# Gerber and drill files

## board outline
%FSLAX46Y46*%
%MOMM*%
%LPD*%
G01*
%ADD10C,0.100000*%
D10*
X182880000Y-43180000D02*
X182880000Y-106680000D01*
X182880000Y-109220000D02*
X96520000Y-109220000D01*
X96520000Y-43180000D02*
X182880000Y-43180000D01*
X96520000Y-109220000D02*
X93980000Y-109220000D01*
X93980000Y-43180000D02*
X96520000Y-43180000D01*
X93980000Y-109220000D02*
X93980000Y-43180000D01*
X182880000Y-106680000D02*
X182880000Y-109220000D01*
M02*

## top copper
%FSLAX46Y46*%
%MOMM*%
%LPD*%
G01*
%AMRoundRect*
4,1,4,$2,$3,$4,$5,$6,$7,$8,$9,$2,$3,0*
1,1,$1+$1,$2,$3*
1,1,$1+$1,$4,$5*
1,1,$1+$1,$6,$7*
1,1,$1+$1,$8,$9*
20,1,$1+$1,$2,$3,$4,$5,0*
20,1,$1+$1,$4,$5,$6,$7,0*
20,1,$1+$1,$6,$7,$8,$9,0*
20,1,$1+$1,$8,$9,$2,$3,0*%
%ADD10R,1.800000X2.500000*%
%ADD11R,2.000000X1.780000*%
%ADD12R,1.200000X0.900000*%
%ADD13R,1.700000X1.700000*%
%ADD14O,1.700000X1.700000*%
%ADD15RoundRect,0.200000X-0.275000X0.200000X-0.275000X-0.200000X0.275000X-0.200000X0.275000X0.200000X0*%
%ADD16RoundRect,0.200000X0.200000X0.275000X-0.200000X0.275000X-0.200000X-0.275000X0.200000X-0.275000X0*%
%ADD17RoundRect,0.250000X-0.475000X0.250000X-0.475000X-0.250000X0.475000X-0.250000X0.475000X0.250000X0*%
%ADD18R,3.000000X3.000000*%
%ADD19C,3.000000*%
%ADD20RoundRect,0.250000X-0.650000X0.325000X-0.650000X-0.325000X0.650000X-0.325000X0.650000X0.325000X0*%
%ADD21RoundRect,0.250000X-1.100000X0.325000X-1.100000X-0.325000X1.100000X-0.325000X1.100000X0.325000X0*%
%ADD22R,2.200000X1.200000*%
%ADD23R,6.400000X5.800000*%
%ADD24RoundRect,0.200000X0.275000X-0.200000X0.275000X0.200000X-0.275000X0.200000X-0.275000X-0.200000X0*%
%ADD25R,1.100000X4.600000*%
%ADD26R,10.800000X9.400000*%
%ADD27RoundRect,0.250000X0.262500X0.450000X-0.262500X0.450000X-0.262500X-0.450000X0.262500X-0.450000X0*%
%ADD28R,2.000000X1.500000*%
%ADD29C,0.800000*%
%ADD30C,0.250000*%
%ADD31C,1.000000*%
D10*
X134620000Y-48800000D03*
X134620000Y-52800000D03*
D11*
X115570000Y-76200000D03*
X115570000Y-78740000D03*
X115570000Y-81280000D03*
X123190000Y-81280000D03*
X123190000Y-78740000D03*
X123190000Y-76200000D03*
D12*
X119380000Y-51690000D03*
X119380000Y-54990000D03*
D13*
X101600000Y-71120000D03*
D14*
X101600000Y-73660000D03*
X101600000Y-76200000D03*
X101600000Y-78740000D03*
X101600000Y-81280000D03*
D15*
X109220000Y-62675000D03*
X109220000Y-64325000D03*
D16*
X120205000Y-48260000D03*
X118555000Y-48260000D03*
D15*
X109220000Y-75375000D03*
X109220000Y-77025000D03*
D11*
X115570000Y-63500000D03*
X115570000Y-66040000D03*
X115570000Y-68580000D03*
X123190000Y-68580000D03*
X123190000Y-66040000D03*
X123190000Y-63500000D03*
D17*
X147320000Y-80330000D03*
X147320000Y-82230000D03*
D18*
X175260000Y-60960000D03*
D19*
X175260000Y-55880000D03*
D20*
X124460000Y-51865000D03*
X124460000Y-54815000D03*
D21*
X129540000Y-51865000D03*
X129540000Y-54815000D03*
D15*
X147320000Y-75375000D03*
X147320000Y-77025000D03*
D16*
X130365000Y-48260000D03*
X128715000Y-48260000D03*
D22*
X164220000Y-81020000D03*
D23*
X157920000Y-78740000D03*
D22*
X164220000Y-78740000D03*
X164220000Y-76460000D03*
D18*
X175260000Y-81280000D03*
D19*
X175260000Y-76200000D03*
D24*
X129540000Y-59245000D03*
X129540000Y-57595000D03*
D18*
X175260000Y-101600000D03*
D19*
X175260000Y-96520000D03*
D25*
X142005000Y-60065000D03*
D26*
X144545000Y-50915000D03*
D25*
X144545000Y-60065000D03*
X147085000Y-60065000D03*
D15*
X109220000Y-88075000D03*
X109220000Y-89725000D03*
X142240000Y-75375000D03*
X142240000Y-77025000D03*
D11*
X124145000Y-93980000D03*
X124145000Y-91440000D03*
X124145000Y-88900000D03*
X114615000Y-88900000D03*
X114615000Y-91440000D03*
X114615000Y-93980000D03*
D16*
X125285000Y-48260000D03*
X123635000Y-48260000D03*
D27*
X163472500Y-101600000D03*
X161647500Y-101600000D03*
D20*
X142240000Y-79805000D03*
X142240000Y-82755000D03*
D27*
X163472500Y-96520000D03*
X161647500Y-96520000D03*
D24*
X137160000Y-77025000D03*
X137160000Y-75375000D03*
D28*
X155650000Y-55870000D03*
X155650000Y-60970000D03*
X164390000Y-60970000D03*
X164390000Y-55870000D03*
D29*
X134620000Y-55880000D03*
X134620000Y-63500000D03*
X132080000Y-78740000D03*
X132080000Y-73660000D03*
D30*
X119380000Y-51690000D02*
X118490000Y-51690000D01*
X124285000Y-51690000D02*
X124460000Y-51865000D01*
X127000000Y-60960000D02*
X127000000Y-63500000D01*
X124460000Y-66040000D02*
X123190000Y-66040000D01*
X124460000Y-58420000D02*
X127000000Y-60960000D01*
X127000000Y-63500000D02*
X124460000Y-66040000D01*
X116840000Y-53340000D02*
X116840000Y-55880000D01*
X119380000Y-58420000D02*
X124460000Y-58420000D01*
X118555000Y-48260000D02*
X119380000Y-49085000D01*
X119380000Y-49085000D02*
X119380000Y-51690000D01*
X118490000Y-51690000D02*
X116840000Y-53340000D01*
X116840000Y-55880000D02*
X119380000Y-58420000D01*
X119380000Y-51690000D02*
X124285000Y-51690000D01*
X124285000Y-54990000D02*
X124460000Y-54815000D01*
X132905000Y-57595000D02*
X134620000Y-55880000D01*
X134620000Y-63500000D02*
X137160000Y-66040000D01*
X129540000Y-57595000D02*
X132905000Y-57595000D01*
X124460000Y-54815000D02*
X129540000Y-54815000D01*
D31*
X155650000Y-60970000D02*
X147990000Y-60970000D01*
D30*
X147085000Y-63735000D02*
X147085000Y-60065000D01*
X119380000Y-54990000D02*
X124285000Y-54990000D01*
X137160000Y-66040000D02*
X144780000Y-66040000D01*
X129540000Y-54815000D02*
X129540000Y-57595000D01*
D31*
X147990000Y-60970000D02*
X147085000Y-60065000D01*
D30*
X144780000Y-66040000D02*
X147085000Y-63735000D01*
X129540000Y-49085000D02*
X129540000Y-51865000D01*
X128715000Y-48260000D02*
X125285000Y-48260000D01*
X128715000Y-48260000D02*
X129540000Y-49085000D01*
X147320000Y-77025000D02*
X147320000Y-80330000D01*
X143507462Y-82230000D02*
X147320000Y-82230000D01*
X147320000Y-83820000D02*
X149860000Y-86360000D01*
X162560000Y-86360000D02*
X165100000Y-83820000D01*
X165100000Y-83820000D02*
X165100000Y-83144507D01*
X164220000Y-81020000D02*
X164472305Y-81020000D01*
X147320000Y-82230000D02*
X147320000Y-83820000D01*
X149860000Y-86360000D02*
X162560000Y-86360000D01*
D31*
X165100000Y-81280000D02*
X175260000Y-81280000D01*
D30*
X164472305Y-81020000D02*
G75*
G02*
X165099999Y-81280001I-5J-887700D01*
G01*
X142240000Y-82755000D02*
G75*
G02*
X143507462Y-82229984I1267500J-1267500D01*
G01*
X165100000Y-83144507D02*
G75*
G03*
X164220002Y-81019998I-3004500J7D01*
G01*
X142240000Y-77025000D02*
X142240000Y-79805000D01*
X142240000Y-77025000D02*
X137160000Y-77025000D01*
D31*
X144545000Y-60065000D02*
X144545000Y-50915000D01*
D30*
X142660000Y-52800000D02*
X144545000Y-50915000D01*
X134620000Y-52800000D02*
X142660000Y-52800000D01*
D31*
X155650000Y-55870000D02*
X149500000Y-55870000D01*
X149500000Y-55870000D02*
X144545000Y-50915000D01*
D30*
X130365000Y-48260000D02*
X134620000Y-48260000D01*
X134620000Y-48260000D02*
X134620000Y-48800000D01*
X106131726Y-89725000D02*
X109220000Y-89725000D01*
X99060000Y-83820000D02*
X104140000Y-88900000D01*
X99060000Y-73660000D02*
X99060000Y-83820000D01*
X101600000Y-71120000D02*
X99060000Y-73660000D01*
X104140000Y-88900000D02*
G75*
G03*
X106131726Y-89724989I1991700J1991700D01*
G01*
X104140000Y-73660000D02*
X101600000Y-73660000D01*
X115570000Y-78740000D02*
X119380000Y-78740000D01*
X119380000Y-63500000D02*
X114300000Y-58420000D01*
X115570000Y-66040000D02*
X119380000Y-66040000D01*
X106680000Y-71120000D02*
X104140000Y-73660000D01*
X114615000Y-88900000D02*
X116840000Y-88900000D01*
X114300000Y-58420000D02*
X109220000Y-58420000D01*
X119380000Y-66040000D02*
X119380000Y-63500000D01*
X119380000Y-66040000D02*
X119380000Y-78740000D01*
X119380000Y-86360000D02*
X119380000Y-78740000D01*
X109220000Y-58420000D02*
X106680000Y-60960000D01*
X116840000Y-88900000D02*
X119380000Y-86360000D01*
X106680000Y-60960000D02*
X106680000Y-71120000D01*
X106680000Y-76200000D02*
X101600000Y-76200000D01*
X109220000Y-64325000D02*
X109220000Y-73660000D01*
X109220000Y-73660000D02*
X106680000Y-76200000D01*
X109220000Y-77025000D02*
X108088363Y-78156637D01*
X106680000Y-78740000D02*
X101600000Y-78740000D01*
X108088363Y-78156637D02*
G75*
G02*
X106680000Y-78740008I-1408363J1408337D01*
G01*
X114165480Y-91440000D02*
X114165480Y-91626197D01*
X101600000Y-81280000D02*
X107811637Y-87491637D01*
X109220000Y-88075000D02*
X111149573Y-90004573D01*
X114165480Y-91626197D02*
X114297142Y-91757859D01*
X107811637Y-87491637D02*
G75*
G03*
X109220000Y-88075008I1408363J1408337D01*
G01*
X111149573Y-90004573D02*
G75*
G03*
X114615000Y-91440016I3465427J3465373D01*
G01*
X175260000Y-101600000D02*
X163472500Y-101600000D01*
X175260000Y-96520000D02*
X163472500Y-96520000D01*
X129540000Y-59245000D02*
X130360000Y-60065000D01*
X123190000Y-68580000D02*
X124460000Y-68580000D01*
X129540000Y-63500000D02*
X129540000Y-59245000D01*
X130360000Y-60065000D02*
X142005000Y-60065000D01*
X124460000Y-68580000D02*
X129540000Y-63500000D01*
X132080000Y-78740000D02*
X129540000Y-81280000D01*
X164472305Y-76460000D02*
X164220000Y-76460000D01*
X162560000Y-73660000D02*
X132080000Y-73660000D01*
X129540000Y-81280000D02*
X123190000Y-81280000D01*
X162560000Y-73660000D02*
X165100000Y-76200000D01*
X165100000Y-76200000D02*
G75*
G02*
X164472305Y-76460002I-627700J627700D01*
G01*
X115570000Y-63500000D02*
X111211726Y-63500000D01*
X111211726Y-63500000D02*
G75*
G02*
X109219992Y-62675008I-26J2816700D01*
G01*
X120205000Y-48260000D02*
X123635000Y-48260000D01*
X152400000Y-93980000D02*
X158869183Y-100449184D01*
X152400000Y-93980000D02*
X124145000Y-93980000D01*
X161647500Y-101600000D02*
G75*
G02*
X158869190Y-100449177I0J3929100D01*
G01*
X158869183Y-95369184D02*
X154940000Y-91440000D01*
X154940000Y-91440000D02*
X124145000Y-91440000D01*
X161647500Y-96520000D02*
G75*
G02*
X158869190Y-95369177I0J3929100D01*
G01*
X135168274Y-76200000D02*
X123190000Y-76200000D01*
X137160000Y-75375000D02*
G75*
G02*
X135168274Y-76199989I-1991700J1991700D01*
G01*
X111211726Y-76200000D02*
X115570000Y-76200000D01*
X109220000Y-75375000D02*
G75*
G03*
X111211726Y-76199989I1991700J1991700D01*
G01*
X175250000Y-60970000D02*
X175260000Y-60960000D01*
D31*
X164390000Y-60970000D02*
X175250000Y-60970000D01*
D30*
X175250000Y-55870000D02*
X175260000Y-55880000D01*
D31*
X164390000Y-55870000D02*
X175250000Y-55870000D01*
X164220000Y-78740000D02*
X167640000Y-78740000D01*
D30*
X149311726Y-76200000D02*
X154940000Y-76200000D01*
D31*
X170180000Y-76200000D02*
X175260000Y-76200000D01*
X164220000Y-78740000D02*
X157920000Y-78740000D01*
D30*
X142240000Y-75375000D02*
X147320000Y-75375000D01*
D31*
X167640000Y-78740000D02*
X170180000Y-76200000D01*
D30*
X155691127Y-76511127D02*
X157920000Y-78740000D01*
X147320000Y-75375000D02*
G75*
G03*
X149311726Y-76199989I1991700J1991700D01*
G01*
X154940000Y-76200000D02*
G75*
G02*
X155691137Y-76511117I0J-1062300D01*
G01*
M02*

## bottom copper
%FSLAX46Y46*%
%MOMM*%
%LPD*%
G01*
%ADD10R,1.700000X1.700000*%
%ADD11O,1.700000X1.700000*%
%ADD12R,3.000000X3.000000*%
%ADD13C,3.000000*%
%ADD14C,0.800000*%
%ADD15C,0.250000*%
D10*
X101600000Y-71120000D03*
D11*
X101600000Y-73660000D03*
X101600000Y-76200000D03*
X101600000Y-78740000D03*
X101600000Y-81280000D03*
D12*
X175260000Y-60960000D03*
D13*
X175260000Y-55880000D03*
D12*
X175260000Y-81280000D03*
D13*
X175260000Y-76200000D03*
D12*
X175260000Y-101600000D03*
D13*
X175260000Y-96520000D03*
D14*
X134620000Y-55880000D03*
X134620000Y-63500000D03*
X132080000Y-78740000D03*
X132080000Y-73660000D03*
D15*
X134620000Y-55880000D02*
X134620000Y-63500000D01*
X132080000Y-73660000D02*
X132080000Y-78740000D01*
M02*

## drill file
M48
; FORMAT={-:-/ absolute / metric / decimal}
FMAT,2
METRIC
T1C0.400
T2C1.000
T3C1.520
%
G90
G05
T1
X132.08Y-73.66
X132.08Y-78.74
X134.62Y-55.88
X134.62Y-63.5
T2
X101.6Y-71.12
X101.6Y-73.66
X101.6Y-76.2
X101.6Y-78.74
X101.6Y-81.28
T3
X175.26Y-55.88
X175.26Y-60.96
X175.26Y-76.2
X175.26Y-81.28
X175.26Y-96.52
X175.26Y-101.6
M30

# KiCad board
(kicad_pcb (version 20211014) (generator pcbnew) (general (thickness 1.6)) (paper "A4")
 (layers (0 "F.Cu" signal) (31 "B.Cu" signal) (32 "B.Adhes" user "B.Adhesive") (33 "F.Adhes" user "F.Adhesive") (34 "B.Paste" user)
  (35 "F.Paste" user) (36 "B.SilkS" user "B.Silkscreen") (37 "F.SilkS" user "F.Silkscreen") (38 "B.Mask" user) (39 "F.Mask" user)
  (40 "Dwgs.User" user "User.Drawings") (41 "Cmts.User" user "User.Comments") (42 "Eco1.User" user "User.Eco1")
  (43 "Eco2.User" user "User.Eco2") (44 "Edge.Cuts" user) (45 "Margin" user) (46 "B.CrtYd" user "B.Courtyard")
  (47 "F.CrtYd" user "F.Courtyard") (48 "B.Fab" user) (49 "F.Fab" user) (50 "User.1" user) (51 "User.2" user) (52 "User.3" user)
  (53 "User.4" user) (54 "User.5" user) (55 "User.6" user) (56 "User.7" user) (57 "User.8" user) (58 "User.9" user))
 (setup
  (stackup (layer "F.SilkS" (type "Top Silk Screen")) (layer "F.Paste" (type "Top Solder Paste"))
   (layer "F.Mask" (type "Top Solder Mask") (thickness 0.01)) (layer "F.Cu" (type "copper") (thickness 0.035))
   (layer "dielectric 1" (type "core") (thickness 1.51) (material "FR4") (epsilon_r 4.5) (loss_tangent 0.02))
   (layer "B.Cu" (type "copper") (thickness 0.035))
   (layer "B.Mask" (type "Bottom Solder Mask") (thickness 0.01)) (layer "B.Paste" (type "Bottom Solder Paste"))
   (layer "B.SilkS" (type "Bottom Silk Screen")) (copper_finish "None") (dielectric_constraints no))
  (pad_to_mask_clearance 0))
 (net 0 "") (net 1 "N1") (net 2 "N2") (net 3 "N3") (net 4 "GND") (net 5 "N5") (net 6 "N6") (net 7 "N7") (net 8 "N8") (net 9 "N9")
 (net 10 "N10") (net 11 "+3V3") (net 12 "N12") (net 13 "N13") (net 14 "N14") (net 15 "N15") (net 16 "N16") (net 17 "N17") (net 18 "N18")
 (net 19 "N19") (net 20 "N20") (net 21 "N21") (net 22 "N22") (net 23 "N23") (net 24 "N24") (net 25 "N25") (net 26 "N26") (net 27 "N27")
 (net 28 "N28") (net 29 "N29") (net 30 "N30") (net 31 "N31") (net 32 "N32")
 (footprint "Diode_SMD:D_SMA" (layer "F.Cu") (at 134.62 50.8 -90)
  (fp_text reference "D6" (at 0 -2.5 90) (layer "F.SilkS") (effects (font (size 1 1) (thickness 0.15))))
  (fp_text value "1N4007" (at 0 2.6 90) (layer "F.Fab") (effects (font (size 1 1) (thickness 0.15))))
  (pad "1" smd rect locked (at -2 0 270) (size 2.5 1.8) (layers "F.Cu" "F.Paste" "F.Mask") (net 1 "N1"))
  (pad "2" smd rect locked (at 2 0 270) (size 2.5 1.8) (layers "F.Cu" "F.Paste" "F.Mask") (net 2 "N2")))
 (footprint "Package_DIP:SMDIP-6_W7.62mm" (layer "F.Cu") (at 119.38 78.74)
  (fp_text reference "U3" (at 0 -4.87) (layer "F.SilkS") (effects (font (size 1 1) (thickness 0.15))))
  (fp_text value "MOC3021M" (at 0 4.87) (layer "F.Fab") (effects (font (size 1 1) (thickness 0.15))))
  (pad "1" smd rect locked (at -3.81 -2.54) (size 2 1.78) (layers "F.Cu" "F.Paste" "F.Mask") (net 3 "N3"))
  (pad "2" smd rect locked (at -3.81 0) (size 2 1.78) (layers "F.Cu" "F.Paste" "F.Mask") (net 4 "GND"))
  (pad "3" smd rect locked (at -3.81 2.54) (size 2 1.78) (layers "F.Cu" "F.Paste" "F.Mask") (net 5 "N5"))
  (pad "4" smd rect locked (at 3.81 2.54) (size 2 1.78) (layers "F.Cu" "F.Paste" "F.Mask") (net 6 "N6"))
  (pad "5" smd rect locked (at 3.81 0) (size 2 1.78) (layers "F.Cu" "F.Paste" "F.Mask") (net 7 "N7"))
  (pad "6" smd rect locked (at 3.81 -2.54) (size 2 1.78) (layers "F.Cu" "F.Paste" "F.Mask") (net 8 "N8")))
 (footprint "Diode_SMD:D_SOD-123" (layer "F.Cu") (at 119.38 53.34 -90)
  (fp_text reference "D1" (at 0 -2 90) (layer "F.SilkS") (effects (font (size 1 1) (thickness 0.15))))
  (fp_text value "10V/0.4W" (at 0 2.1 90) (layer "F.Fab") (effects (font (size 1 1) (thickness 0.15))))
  (pad "1" smd rect locked (at -1.65 0 270) (size 0.9 1.2) (layers "F.Cu" "F.Paste" "F.Mask") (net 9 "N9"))
  (pad "2" smd rect locked (at 1.65 0 270) (size 0.9 1.2) (layers "F.Cu" "F.Paste" "F.Mask") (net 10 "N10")))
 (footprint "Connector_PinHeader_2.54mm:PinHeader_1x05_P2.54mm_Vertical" (layer "F.Cu") (at 101.6 71.12)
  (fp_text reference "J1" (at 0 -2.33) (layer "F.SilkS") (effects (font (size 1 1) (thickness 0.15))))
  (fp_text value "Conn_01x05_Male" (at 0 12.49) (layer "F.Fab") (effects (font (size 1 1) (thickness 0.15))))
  (pad "1" thru_hole rect locked (at 0 0) (size 1.7 1.7) (drill 1) (layers *.Cu *.Mask) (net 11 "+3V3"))
  (pad "2" thru_hole oval locked (at 0 2.54) (size 1.7 1.7) (drill 1) (layers *.Cu *.Mask) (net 4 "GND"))
  (pad "3" thru_hole oval locked (at 0 5.08) (size 1.7 1.7) (drill 1) (layers *.Cu *.Mask) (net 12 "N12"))
  (pad "4" thru_hole oval locked (at 0 7.62) (size 1.7 1.7) (drill 1) (layers *.Cu *.Mask) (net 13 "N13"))
  (pad "5" thru_hole oval locked (at 0 10.16) (size 1.7 1.7) (drill 1) (layers *.Cu *.Mask) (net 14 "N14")))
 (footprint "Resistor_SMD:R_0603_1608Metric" (layer "F.Cu") (at 109.22 63.5 -90)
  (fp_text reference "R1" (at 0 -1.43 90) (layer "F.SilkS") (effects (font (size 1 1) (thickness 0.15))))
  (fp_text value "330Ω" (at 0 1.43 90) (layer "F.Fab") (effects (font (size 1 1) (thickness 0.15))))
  (pad "1" smd roundrect locked (at -0.825 0 270) (size 0.8 0.95) (layers "F.Cu" "F.Paste" "F.Mask") (roundrect_rratio 0.25) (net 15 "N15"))
  (pad "2" smd roundrect locked (at 0.825 0 270) (size 0.8 0.95) (layers "F.Cu" "F.Paste" "F.Mask") (roundrect_rratio 0.25) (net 12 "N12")))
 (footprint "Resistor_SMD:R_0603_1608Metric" (layer "F.Cu") (at 119.38 48.26 180)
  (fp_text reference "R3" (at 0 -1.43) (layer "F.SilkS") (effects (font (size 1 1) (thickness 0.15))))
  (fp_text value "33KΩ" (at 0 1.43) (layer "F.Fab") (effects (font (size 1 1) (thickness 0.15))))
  (pad "1" smd roundrect locked (at -0.825 0 180) (size 0.8 0.95) (layers "F.Cu" "F.Paste" "F.Mask") (roundrect_rratio 0.25) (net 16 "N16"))
  (pad "2" smd roundrect locked (at 0.825 0 180) (size 0.8 0.95) (layers "F.Cu" "F.Paste" "F.Mask") (roundrect_rratio 0.25) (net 9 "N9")))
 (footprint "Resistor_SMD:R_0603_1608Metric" (layer "F.Cu") (at 109.22 76.2 -90)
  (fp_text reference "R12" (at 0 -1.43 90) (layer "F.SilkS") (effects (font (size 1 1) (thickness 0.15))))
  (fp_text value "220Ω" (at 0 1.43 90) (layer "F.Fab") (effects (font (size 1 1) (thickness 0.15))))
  (pad "1" smd roundrect locked (at -0.825 0 270) (size 0.8 0.95) (layers "F.Cu" "F.Paste" "F.Mask") (roundrect_rratio 0.25) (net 3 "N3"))
  (pad "2" smd roundrect locked (at 0.825 0 270) (size 0.8 0.95) (layers "F.Cu" "F.Paste" "F.Mask") (roundrect_rratio 0.25) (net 13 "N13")))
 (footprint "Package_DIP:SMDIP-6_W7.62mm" (layer "F.Cu") (at 119.38 66.04)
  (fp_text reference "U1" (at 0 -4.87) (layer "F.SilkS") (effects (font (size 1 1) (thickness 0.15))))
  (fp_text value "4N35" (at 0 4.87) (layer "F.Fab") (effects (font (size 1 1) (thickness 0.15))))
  (pad "1" smd rect locked (at -3.81 -2.54) (size 2 1.78) (layers "F.Cu" "F.Paste" "F.Mask") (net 15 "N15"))
  (pad "2" smd rect locked (at -3.81 0) (size 2 1.78) (layers "F.Cu" "F.Paste" "F.Mask") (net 4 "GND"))
  (pad "3" smd rect locked (at -3.81 2.54) (size 2 1.78) (layers "F.Cu" "F.Paste" "F.Mask") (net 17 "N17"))
  (pad "4" smd rect locked (at 3.81 2.54) (size 2 1.78) (layers "F.Cu" "F.Paste" "F.Mask") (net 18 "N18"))
  (pad "5" smd rect locked (at 3.81 0) (size 2 1.78) (layers "F.Cu" "F.Paste" "F.Mask") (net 9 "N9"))
  (pad "6" smd rect locked (at 3.81 -2.54) (size 2 1.78) (layers "F.Cu" "F.Paste" "F.Mask") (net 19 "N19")))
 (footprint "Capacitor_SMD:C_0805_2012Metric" (layer "F.Cu") (at 147.32 81.28 -90)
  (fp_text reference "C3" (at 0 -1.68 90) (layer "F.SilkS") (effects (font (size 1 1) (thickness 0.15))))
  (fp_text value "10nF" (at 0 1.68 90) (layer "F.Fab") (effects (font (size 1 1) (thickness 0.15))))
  (pad "1" smd roundrect locked (at -0.95 0 270) (size 1 1.45) (layers "F.Cu" "F.Paste" "F.Mask") (roundrect_rratio 0.25) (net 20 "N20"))
  (pad "2" smd roundrect locked (at 0.95 0 270) (size 1 1.45) (layers "F.Cu" "F.Paste" "F.Mask") (roundrect_rratio 0.25) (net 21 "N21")))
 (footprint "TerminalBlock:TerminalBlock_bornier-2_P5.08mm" (layer "F.Cu") (at 175.26 60.96 90)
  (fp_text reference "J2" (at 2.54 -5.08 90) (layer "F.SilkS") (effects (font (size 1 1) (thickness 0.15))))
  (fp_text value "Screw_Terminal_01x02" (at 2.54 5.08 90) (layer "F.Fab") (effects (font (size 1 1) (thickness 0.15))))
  (pad "1" thru_hole rect locked (at 0 0 90) (size 3 3) (drill 1.52) (layers *.Cu *.Mask) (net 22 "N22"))
  (pad "2" thru_hole circle locked (at 5.08 0 90) (size 3 3) (drill 1.52) (layers *.Cu *.Mask) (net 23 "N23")))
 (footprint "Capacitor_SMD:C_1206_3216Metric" (layer "F.Cu") (at 124.46 53.34 -90)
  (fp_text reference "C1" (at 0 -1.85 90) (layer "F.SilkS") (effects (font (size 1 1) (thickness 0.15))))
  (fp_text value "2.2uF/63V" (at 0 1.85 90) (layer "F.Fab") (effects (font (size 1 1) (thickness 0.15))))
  (pad "1" smd roundrect locked (at -1.475 0 270) (size 1.15 1.8) (layers "F.Cu" "F.Paste" "F.Mask") (roundrect_rratio 0.2173913043)
   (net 9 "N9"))
  (pad "2" smd roundrect locked (at 1.475 0 270) (size 1.15 1.8) (layers "F.Cu" "F.Paste" "F.Mask") (roundrect_rratio 0.2173913043)
   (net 10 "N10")))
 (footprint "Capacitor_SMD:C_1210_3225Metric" (layer "F.Cu") (at 129.54 53.34 -90)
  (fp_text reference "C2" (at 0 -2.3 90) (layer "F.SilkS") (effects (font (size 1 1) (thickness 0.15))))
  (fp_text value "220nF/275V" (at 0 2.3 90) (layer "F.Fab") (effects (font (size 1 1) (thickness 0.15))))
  (pad "1" smd roundrect locked (at -1.475 0 270) (size 1.15 2.7) (layers "F.Cu" "F.Paste" "F.Mask") (roundrect_rratio 0.2173913043)
   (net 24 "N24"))
  (pad "2" smd roundrect locked (at 1.475 0 270) (size 1.15 2.7) (layers "F.Cu" "F.Paste" "F.Mask") (roundrect_rratio 0.2173913043)
   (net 10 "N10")))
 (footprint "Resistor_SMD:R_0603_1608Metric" (layer "F.Cu") (at 147.32 76.2 -90)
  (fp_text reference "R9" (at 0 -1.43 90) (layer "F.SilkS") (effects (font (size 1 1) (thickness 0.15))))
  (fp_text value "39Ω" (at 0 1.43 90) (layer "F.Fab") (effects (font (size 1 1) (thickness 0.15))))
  (pad "1" smd roundrect locked (at -0.825 0 270) (size 0.8 0.95) (layers "F.Cu" "F.Paste" "F.Mask") (roundrect_rratio 0.25) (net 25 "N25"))
  (pad "2" smd roundrect locked (at 0.825 0 270) (size 0.8 0.95) (layers "F.Cu" "F.Paste" "F.Mask") (roundrect_rratio 0.25) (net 20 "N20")))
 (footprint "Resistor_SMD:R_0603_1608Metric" (layer "F.Cu") (at 129.54 48.26 180)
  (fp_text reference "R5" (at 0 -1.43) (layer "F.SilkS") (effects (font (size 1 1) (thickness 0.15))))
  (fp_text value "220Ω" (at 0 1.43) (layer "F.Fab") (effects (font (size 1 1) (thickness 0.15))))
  (pad "1" smd roundrect locked (at -0.825 0 180) (size 0.8 0.95) (layers "F.Cu" "F.Paste" "F.Mask") (roundrect_rratio 0.25) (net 1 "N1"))
  (pad "2" smd roundrect locked (at 0.825 0 180) (size 0.8 0.95) (layers "F.Cu" "F.Paste" "F.Mask") (roundrect_rratio 0.25) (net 24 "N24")))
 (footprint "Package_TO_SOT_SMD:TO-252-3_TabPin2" (layer "F.Cu") (at 160.02 78.74 180)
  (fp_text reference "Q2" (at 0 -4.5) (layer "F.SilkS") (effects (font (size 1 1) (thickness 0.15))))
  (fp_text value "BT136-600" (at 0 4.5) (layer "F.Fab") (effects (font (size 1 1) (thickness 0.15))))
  (pad "" smd rect locked (at 0.425 1.525 180) (size 3.05 2.75) (layers "F.Paste"))
  (pad "" smd rect locked (at 3.775 -1.525 180) (size 3.05 2.75) (layers "F.Paste"))
  (pad "" smd rect locked (at 0.425 -1.525 180) (size 3.05 2.75) (layers "F.Paste"))
  (pad "" smd rect locked (at 3.775 1.525 180) (size 3.05 2.75) (layers "F.Paste"))
  (pad "1" smd rect locked (at -4.2 -2.28 180) (size 2.2 1.2) (layers "F.Cu" "F.Paste" "F.Mask") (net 21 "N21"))
  (pad "2" smd rect locked (at 2.1 0 180) (size 6.4 5.8) (layers "F.Cu" "F.Mask") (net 25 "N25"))
  (pad "2" smd rect locked (at -4.2 0 180) (size 2.2 1.2) (layers "F.Cu" "F.Paste" "F.Mask") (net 25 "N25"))
  (pad "3" smd rect locked (at -4.2 2.28 180) (size 2.2 1.2) (layers "F.Cu" "F.Paste" "F.Mask") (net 6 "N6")))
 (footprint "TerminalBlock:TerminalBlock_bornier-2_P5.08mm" (layer "F.Cu") (at 175.26 81.28 90)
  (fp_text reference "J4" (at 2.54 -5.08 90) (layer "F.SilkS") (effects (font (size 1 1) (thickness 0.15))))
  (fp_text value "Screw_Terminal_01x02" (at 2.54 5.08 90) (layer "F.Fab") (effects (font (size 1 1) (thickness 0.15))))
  (pad "1" thru_hole rect locked (at 0 0 90) (size 3 3) (drill 1.52) (layers *.Cu *.Mask) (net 21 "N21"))
  (pad "2" thru_hole circle locked (at 5.08 0 90) (size 3 3) (drill 1.52) (layers *.Cu *.Mask) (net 25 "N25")))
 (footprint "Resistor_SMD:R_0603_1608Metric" (layer "F.Cu") (at 129.54 58.42 90)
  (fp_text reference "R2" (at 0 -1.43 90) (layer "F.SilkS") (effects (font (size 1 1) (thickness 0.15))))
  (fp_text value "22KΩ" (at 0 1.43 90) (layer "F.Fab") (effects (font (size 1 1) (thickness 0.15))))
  (pad "1" smd roundrect locked (at -0.825 0 90) (size 0.8 0.95) (layers "F.Cu" "F.Paste" "F.Mask") (roundrect_rratio 0.25) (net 18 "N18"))
  (pad "2" smd roundrect locked (at 0.825 0 90) (size 0.8 0.95) (layers "F.Cu" "F.Paste" "F.Mask") (roundrect_rratio 0.25) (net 10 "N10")))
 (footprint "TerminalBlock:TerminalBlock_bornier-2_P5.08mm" (layer "F.Cu") (at 175.26 101.6 90)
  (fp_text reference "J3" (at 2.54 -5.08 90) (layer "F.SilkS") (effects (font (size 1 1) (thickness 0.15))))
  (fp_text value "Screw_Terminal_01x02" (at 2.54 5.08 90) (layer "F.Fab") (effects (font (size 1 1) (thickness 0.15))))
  (pad "1" thru_hole rect locked (at 0 0 90) (size 3 3) (drill 1.52) (layers *.Cu *.Mask) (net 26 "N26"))
  (pad "2" thru_hole circle locked (at 5.08 0 90) (size 3 3) (drill 1.52) (layers *.Cu *.Mask) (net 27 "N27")))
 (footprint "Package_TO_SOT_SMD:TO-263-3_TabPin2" (layer "F.Cu") (at 144.545 54.29 90)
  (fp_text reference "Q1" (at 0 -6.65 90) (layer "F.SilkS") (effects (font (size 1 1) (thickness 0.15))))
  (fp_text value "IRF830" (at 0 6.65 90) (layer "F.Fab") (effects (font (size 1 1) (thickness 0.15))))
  (pad "" smd rect locked (at 5.8 2.775 90) (size 4.55 5.25) (layers "F.Paste"))
  (pad "" smd rect locked (at 0.95 -2.775 90) (size 4.55 5.25) (layers "F.Paste"))
  (pad "" smd rect locked (at 0.95 2.775 90) (size 4.55 5.25) (layers "F.Paste"))
  (pad "" smd rect locked (at 5.8 -2.775 90) (size 4.55 5.25) (layers "F.Paste"))
  (pad "1" smd rect locked (at -5.775 -2.54 90) (size 4.6 1.1) (layers "F.Cu" "F.Paste" "F.Mask") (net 18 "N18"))
  (pad "2" smd rect locked (at 3.375 0 90) (size 9.4 10.8) (layers "F.Cu" "F.Mask") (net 2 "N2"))
  (pad "2" smd rect locked (at -5.775 0 90) (size 4.6 1.1) (layers "F.Cu" "F.Paste" "F.Mask") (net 2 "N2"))
  (pad "3" smd rect locked (at -5.775 2.54 90) (size 4.6 1.1) (layers "F.Cu" "F.Paste" "F.Mask") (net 10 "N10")))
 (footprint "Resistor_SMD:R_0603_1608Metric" (layer "F.Cu") (at 109.22 88.9 -90)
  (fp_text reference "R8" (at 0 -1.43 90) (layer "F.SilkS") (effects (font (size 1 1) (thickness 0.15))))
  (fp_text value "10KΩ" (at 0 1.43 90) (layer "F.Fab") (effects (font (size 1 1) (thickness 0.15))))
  (pad "1" smd roundrect locked (at -0.825 0 270) (size 0.8 0.95) (layers "F.Cu" "F.Paste" "F.Mask") (roundrect_rratio 0.25) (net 14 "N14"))
  (pad "2" smd roundrect locked (at 0.825 0 270) (size 0.8 0.95) (layers "F.Cu" "F.Paste" "F.Mask") (roundrect_rratio 0.25) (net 11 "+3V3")))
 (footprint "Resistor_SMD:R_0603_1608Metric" (layer "F.Cu") (at 142.24 76.2 -90)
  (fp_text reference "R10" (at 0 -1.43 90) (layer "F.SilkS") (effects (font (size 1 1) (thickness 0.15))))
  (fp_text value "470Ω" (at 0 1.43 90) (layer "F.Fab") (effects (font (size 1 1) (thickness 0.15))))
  (pad "1" smd roundrect locked (at -0.825 0 270) (size 0.8 0.95) (layers "F.Cu" "F.Paste" "F.Mask") (roundrect_rratio 0.25) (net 25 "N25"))
  (pad "2" smd roundrect locked (at 0.825 0 270) (size 0.8 0.95) (layers "F.Cu" "F.Paste" "F.Mask") (roundrect_rratio 0.25) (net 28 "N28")))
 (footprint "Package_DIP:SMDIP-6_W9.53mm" (layer "F.Cu") (at 119.38 91.44 180)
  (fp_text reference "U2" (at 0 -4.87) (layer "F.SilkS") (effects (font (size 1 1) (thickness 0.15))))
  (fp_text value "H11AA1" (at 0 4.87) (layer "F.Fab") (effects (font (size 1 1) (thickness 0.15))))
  (pad "1" smd rect locked (at -4.765 -2.54 180) (size 2 1.78) (layers "F.Cu" "F.Paste" "F.Mask") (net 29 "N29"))
  (pad "2" smd rect locked (at -4.765 0 180) (size 2 1.78) (layers "F.Cu" "F.Paste" "F.Mask") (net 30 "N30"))
  (pad "3" smd rect locked (at -4.765 2.54 180) (size 2 1.78) (layers "F.Cu" "F.Paste" "F.Mask") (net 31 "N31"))
  (pad "4" smd rect locked (at 4.765 2.54 180) (size 2 1.78) (layers "F.Cu" "F.Paste" "F.Mask") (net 4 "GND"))
  (pad "5" smd rect locked (at 4.765 0 180) (size 2 1.78) (layers "F.Cu" "F.Paste" "F.Mask") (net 14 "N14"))
  (pad "6" smd rect locked (at 4.765 -2.54 180) (size 2 1.78) (layers "F.Cu" "F.Paste" "F.Mask") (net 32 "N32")))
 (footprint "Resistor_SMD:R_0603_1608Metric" (layer "F.Cu") (at 124.46 48.26 180)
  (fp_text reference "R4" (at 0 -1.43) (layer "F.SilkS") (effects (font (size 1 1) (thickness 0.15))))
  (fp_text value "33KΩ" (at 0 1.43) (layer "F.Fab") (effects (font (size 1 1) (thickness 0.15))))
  (pad "1" smd roundrect locked (at -0.825 0 180) (size 0.8 0.95) (layers "F.Cu" "F.Paste" "F.Mask") (roundrect_rratio 0.25) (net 24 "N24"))
  (pad "2" smd roundrect locked (at 0.825 0 180) (size 0.8 0.95) (layers "F.Cu" "F.Paste" "F.Mask") (roundrect_rratio 0.25) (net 16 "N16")))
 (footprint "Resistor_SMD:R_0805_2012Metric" (layer "F.Cu") (at 162.56 101.6 180)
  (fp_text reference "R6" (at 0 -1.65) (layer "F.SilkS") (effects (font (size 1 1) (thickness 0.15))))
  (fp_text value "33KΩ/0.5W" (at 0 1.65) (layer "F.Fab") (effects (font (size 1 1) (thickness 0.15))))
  (pad "1" smd roundrect locked (at -0.9125 0 180) (size 1.025 1.4) (layers "F.Cu" "F.Paste" "F.Mask") (roundrect_rratio 0.243902439)
   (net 26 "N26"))
  (pad "2" smd roundrect locked (at 0.9125 0 180) (size 1.025 1.4) (layers "F.Cu" "F.Paste" "F.Mask") (roundrect_rratio 0.243902439)
   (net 29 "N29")))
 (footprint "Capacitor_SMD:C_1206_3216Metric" (layer "F.Cu") (at 142.24 81.28 -90)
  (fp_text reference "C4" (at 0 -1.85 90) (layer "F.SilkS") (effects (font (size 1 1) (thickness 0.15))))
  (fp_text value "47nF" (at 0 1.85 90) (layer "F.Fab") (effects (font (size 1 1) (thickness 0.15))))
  (pad "1" smd roundrect locked (at -1.475 0 270) (size 1.15 1.8) (layers "F.Cu" "F.Paste" "F.Mask") (roundrect_rratio 0.2173913043)
   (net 28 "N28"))
  (pad "2" smd roundrect locked (at 1.475 0 270) (size 1.15 1.8) (layers "F.Cu" "F.Paste" "F.Mask") (roundrect_rratio 0.2173913043)
   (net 21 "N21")))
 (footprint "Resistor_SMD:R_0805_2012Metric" (layer "F.Cu") (at 162.56 96.52 180)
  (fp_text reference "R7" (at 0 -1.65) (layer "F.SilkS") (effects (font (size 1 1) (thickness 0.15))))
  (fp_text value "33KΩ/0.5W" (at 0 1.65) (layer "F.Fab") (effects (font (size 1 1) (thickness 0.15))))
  (pad "1" smd roundrect locked (at -0.9125 0 180) (size 1.025 1.4) (layers "F.Cu" "F.Paste" "F.Mask") (roundrect_rratio 0.243902439)
   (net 27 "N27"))
  (pad "2" smd roundrect locked (at 0.9125 0 180) (size 1.025 1.4) (layers "F.Cu" "F.Paste" "F.Mask") (roundrect_rratio 0.243902439)
   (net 30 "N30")))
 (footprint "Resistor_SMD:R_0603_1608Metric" (layer "F.Cu") (at 137.16 76.2 90)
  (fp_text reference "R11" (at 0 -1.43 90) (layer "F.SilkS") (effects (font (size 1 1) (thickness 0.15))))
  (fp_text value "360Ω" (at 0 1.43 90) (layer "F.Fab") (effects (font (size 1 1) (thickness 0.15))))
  (pad "1" smd roundrect locked (at -0.825 0 90) (size 0.8 0.95) (layers "F.Cu" "F.Paste" "F.Mask") (roundrect_rratio 0.25) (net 28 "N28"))
  (pad "2" smd roundrect locked (at 0.825 0 90) (size 0.8 0.95) (layers "F.Cu" "F.Paste" "F.Mask") (roundrect_rratio 0.25) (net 8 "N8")))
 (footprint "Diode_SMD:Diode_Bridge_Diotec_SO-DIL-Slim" (layer "F.Cu") (at 160.02 58.42)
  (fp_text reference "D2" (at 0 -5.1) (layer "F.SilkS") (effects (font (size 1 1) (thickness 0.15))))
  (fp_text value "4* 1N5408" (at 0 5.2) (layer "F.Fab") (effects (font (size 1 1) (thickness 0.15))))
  (pad "1" smd rect locked (at -4.37 -2.55) (size 2 1.5) (layers "F.Cu" "F.Paste" "F.Mask") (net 2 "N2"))
  (pad "2" smd rect locked (at -4.37 2.55) (size 2 1.5) (layers "F.Cu" "F.Paste" "F.Mask") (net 10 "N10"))
  (pad "3" smd rect locked (at 4.37 2.55) (size 2 1.5) (layers "F.Cu" "F.Paste" "F.Mask") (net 22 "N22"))
  (pad "4" smd rect locked (at 4.37 -2.55) (size 2 1.5) (layers "F.Cu" "F.Paste" "F.Mask") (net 23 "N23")))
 (gr_line (start 182.88 43.18) (end 182.88 106.68) (layer "Edge.Cuts") (width 0.1))
 (gr_line (start 182.88 109.22) (end 96.52 109.22) (layer "Edge.Cuts") (width 0.1))
 (gr_line (start 96.52 43.18) (end 182.88 43.18) (layer "Edge.Cuts") (width 0.1))
 (gr_line (start 96.52 109.22) (end 93.98 109.22) (layer "Edge.Cuts") (width 0.1))
 (gr_line (start 93.98 43.18) (end 96.52 43.18) (layer "Edge.Cuts") (width 0.1))
 (gr_line (start 93.98 109.22) (end 93.98 43.18) (layer "Edge.Cuts") (width 0.1))
 (gr_line (start 182.88 106.68) (end 182.88 109.22) (layer "Edge.Cuts") (width 0.1))
 (segment (start 119.38 51.69) (end 118.49 51.69) (width 0.25) (layer "F.Cu") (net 9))
 (segment (start 124.285 51.69) (end 124.46 51.865) (width 0.25) (layer "F.Cu") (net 9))
 (segment (start 127 60.96) (end 127 63.5) (width 0.25) (layer "F.Cu") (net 9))
 (segment (start 124.46 66.04) (end 123.19 66.04) (width 0.25) (layer "F.Cu") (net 9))
 (segment (start 124.46 58.42) (end 127 60.96) (width 0.25) (layer "F.Cu") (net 9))
 (segment (start 127 63.5) (end 124.46 66.04) (width 0.25) (layer "F.Cu") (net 9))
 (segment (start 116.84 53.34) (end 116.84 55.88) (width 0.25) (layer "F.Cu") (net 9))
 (segment (start 119.38 58.42) (end 124.46 58.42) (width 0.25) (layer "F.Cu") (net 9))
 (segment (start 118.555 48.26) (end 119.38 49.085) (width 0.25) (layer "F.Cu") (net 9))
 (segment (start 119.38 49.085) (end 119.38 51.69) (width 0.25) (layer "F.Cu") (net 9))
 (segment (start 118.49 51.69) (end 116.84 53.34) (width 0.25) (layer "F.Cu") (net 9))
 (segment (start 116.84 55.88) (end 119.38 58.42) (width 0.25) (layer "F.Cu") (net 9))
 (segment (start 119.38 51.69) (end 124.285 51.69) (width 0.25) (layer "F.Cu") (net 9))
 (segment (start 124.285 54.99) (end 124.46 54.815) (width 0.25) (layer "F.Cu") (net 10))
 (segment (start 132.905 57.595) (end 134.62 55.88) (width 0.25) (layer "F.Cu") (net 10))
 (segment (start 134.62 63.5) (end 137.16 66.04) (width 0.25) (layer "F.Cu") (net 10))
 (segment (start 129.54 57.595) (end 132.905 57.595) (width 0.25) (layer "F.Cu") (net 10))
 (segment (start 124.46 54.815) (end 129.54 54.815) (width 0.25) (layer "F.Cu") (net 10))
 (segment (start 155.65 60.97) (end 147.99 60.97) (width 1) (layer "F.Cu") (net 10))
 (segment (start 147.085 63.735) (end 147.085 60.065) (width 0.25) (layer "F.Cu") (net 10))
 (segment (start 119.38 54.99) (end 124.285 54.99) (width 0.25) (layer "F.Cu") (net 10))
 (segment (start 137.16 66.04) (end 144.78 66.04) (width 0.25) (layer "F.Cu") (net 10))
 (segment (start 129.54 54.815) (end 129.54 57.595) (width 0.25) (layer "F.Cu") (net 10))
 (segment (start 147.99 60.97) (end 147.085 60.065) (width 1) (layer "F.Cu") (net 10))
 (segment (start 144.78 66.04) (end 147.085 63.735) (width 0.25) (layer "F.Cu") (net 10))
 (via (at 134.62 55.88) (size 0.8) (drill 0.4) (layers "F.Cu" "B.Cu") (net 10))
 (via (at 134.62 63.5) (size 0.8) (drill 0.4) (layers "F.Cu" "B.Cu") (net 10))
 (segment (start 134.62 55.88) (end 134.62 63.5) (width 0.25) (layer "B.Cu") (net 10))
 (segment (start 129.54 49.085) (end 129.54 51.865) (width 0.25) (layer "F.Cu") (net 24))
 (segment (start 128.715 48.26) (end 125.285 48.26) (width 0.25) (layer "F.Cu") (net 24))
 (segment (start 128.715 48.26) (end 129.54 49.085) (width 0.25) (layer "F.Cu") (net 24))
 (segment (start 147.32 77.025) (end 147.32 80.33) (width 0.25) (layer "F.Cu") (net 20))
 (segment (start 143.507462 82.23) (end 147.32 82.23) (width 0.25) (layer "F.Cu") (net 21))
 (segment (start 147.32 83.82) (end 149.86 86.36) (width 0.25) (layer "F.Cu") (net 21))
 (segment (start 162.56 86.36) (end 165.1 83.82) (width 0.25) (layer "F.Cu") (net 21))
 (segment (start 165.1 83.82) (end 165.1 83.144507) (width 0.25) (layer "F.Cu") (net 21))
 (segment (start 164.22 81.02) (end 164.472305 81.02) (width 0.25) (layer "F.Cu") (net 21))
 (segment (start 147.32 82.23) (end 147.32 83.82) (width 0.25) (layer "F.Cu") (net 21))
 (segment (start 149.86 86.36) (end 162.56 86.36) (width 0.25) (layer "F.Cu") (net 21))
 (segment (start 165.1 81.28) (end 175.26 81.28) (width 1) (layer "F.Cu") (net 21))
 (arc (start 164.472305 81.02) (mid 164.812011 81.087572) (end 165.1 81.28) (width 0.25) (layer "F.Cu") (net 21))
 (arc (start 142.24 82.755) (mid 142.821516 82.366443) (end 143.507462 82.23) (width 0.25) (layer "F.Cu") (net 21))
 (arc (start 165.1 83.144507) (mid 164.871296 81.994733) (end 164.22 81.02) (width 0.25) (layer "F.Cu") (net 21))
 (segment (start 142.24 77.025) (end 142.24 79.805) (width 0.25) (layer "F.Cu") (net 28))
 (segment (start 142.24 77.025) (end 137.16 77.025) (width 0.25) (layer "F.Cu") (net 28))
 (segment (start 144.545 60.065) (end 144.545 50.915) (width 1) (layer "F.Cu") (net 2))
 (segment (start 142.66 52.8) (end 144.545 50.915) (width 0.25) (layer "F.Cu") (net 2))
 (segment (start 134.62 52.8) (end 142.66 52.8) (width 0.25) (layer "F.Cu") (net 2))
 (segment (start 155.65 55.87) (end 149.5 55.87) (width 1) (layer "F.Cu") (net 2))
 (segment (start 149.5 55.87) (end 144.545 50.915) (width 1) (layer "F.Cu") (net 2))
 (segment (start 130.365 48.26) (end 134.62 48.26) (width 0.25) (layer "F.Cu") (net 1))
 (segment (start 134.62 48.26) (end 134.62 48.8) (width 0.25) (layer "F.Cu") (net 1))
 (segment (start 106.131726 89.725) (end 109.22 89.725) (width 0.25) (layer "F.Cu") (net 11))
 (segment (start 99.06 83.82) (end 104.14 88.9) (width 0.25) (layer "F.Cu") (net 11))
 (segment (start 99.06 73.66) (end 99.06 83.82) (width 0.25) (layer "F.Cu") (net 11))
 (segment (start 101.6 71.12) (end 99.06 73.66) (width 0.25) (layer "F.Cu") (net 11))
 (arc (start 104.14 88.9) (mid 105.053811 89.51059) (end 106.131726 89.725) (width 0.25) (layer "F.Cu") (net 11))
 (segment (start 104.14 73.66) (end 101.6 73.66) (width 0.25) (layer "F.Cu") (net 4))
 (segment (start 115.57 78.74) (end 119.38 78.74) (width 0.25) (layer "F.Cu") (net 4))
 (segment (start 119.38 63.5) (end 114.3 58.42) (width 0.25) (layer "F.Cu") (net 4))
 (segment (start 115.57 66.04) (end 119.38 66.04) (width 0.25) (layer "F.Cu") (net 4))
 (segment (start 106.68 71.12) (end 104.14 73.66) (width 0.25) (layer "F.Cu") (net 4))
 (segment (start 114.615 88.9) (end 116.84 88.9) (width 0.25) (layer "F.Cu") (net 4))
 (segment (start 114.3 58.42) (end 109.22 58.42) (width 0.25) (layer "F.Cu") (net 4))
 (segment (start 119.38 66.04) (end 119.38 63.5) (width 0.25) (layer "F.Cu") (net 4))
 (segment (start 119.38 66.04) (end 119.38 78.74) (width 0.25) (layer "F.Cu") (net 4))
 (segment (start 119.38 86.36) (end 119.38 78.74) (width 0.25) (layer "F.Cu") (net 4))
 (segment (start 109.22 58.42) (end 106.68 60.96) (width 0.25) (layer "F.Cu") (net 4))
 (segment (start 116.84 88.9) (end 119.38 86.36) (width 0.25) (layer "F.Cu") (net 4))
 (segment (start 106.68 60.96) (end 106.68 71.12) (width 0.25) (layer "F.Cu") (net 4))
 (segment (start 106.68 76.2) (end 101.6 76.2) (width 0.25) (layer "F.Cu") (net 12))
 (segment (start 109.22 64.325) (end 109.22 73.66) (width 0.25) (layer "F.Cu") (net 12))
 (segment (start 109.22 73.66) (end 106.68 76.2) (width 0.25) (layer "F.Cu") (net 12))
 (segment (start 109.22 77.025) (end 108.088363 78.156637) (width 0.25) (layer "F.Cu") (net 13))
 (segment (start 106.68 78.74) (end 101.6 78.74) (width 0.25) (layer "F.Cu") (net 13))
 (arc (start 108.088363 78.156637) (mid 107.442201 78.588389) (end 106.68 78.74) (width 0.25) (layer "F.Cu") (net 13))
 (segment (start 114.16548 91.44) (end 114.16548 91.626197) (width 0.25) (layer "F.Cu") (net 14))
 (segment (start 101.6 81.28) (end 107.811637 87.491637) (width 0.25) (layer "F.Cu") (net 14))
 (segment (start 109.22 88.075) (end 111.149573 90.004573) (width 0.25) (layer "F.Cu") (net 14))
 (segment (start 114.16548 91.626197) (end 114.297142 91.757859) (width 0.25) (layer "F.Cu") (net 14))
 (arc (start 107.811637 87.491637) (mid 108.457799 87.923389) (end 109.22 88.075) (width 0.25) (layer "F.Cu") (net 14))
 (arc (start 111.149573 90.004573) (mid 112.739524 91.066945) (end 114.615 91.44) (width 0.25) (layer "F.Cu") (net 14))
 (segment (start 175.26 101.6) (end 163.4725 101.6) (width 0.25) (layer "F.Cu") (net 26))
 (segment (start 175.26 96.52) (end 163.4725 96.52) (width 0.25) (layer "F.Cu") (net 27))
 (segment (start 129.54 59.245) (end 130.36 60.065) (width 0.25) (layer "F.Cu") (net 18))
 (segment (start 123.19 68.58) (end 124.46 68.58) (width 0.25) (layer "F.Cu") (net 18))
 (segment (start 129.54 63.5) (end 129.54 59.245) (width 0.25) (layer "F.Cu") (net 18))
 (segment (start 130.36 60.065) (end 142.005 60.065) (width 0.25) (layer "F.Cu") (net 18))
 (segment (start 124.46 68.58) (end 129.54 63.5) (width 0.25) (layer "F.Cu") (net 18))
 (segment (start 132.08 78.74) (end 129.54 81.28) (width 0.25) (layer "F.Cu") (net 6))
 (segment (start 164.472305 76.46) (end 164.22 76.46) (width 0.25) (layer "F.Cu") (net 6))
 (segment (start 162.56 73.66) (end 132.08 73.66) (width 0.25) (layer "F.Cu") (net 6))
 (segment (start 129.54 81.28) (end 123.19 81.28) (width 0.25) (layer "F.Cu") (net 6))
 (segment (start 162.56 73.66) (end 165.1 76.2) (width 0.25) (layer "F.Cu") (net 6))
 (via (at 132.08 78.74) (size 0.8) (drill 0.4) (layers "F.Cu" "B.Cu") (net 6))
 (via (at 132.08 73.66) (size 0.8) (drill 0.4) (layers "F.Cu" "B.Cu") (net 6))
 (arc (start 165.1 76.2) (mid 164.812011 76.392428) (end 164.472305 76.46) (width 0.25) (layer "F.Cu") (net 6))
 (segment (start 132.08 73.66) (end 132.08 78.74) (width 0.25) (layer "B.Cu") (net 6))
 (segment (start 115.57 63.5) (end 111.211726 63.5) (width 0.25) (layer "F.Cu") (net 15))
 (arc (start 111.211726 63.5) (mid 110.133812 63.28559) (end 109.22 62.675) (width 0.25) (layer "F.Cu") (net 15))
 (segment (start 120.205 48.26) (end 123.635 48.26) (width 0.25) (layer "F.Cu") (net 16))
 (segment (start 152.4 93.98) (end 158.869183 100.449184) (width 0.25) (layer "F.Cu") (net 29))
 (segment (start 152.4 93.98) (end 124.145 93.98) (width 0.25) (layer "F.Cu") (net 29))
 (arc (start 161.6475 101.6) (mid 160.143886 101.300913) (end 158.869183 100.449184) (width 0.25) (layer "F.Cu") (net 29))
 (segment (start 158.869183 95.369184) (end 154.94 91.44) (width 0.25) (layer "F.Cu") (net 30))
 (segment (start 154.94 91.44) (end 124.145 91.44) (width 0.25) (layer "F.Cu") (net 30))
 (arc (start 161.6475 96.52) (mid 160.143886 96.220913) (end 158.869183 95.369184) (width 0.25) (layer "F.Cu") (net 30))
 (segment (start 135.168274 76.2) (end 123.19 76.2) (width 0.25) (layer "F.Cu") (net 8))
 (arc (start 137.16 75.375) (mid 136.246188 75.985589) (end 135.168274 76.2) (width 0.25) (layer "F.Cu") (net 8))
 (segment (start 111.211726 76.2) (end 115.57 76.2) (width 0.25) (layer "F.Cu") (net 3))
 (arc (start 109.22 75.375) (mid 110.133811 75.98559) (end 111.211726 76.2) (width 0.25) (layer "F.Cu") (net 3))
 (segment (start 175.25 60.97) (end 175.26 60.96) (width 0.25) (layer "F.Cu") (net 22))
 (segment (start 164.39 60.97) (end 175.25 60.97) (width 1) (layer "F.Cu") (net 22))
 (segment (start 175.25 55.87) (end 175.26 55.88) (width 0.25) (layer "F.Cu") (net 23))
 (segment (start 164.39 55.87) (end 175.25 55.87) (width 1) (layer "F.Cu") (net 23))
 (segment (start 164.22 78.74) (end 167.64 78.74) (width 1) (layer "F.Cu") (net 25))
 (segment (start 149.311726 76.2) (end 154.94 76.2) (width 0.25) (layer "F.Cu") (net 25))
 (segment (start 170.18 76.2) (end 175.26 76.2) (width 1) (layer "F.Cu") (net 25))
 (segment (start 164.22 78.74) (end 157.92 78.74) (width 1) (layer "F.Cu") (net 25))
 (segment (start 142.24 75.375) (end 147.32 75.375) (width 0.25) (layer "F.Cu") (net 25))
 (segment (start 167.64 78.74) (end 170.18 76.2) (width 1) (layer "F.Cu") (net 25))
 (segment (start 155.691127 76.511127) (end 157.92 78.74) (width 0.25) (layer "F.Cu") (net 25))
 (arc (start 147.32 75.375) (mid 148.233811 75.98559) (end 149.311726 76.2) (width 0.25) (layer "F.Cu") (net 25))
 (arc (start 154.94 76.2) (mid 155.346507 76.280859) (end 155.691127 76.511127) (width 0.25) (layer "F.Cu") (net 25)))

